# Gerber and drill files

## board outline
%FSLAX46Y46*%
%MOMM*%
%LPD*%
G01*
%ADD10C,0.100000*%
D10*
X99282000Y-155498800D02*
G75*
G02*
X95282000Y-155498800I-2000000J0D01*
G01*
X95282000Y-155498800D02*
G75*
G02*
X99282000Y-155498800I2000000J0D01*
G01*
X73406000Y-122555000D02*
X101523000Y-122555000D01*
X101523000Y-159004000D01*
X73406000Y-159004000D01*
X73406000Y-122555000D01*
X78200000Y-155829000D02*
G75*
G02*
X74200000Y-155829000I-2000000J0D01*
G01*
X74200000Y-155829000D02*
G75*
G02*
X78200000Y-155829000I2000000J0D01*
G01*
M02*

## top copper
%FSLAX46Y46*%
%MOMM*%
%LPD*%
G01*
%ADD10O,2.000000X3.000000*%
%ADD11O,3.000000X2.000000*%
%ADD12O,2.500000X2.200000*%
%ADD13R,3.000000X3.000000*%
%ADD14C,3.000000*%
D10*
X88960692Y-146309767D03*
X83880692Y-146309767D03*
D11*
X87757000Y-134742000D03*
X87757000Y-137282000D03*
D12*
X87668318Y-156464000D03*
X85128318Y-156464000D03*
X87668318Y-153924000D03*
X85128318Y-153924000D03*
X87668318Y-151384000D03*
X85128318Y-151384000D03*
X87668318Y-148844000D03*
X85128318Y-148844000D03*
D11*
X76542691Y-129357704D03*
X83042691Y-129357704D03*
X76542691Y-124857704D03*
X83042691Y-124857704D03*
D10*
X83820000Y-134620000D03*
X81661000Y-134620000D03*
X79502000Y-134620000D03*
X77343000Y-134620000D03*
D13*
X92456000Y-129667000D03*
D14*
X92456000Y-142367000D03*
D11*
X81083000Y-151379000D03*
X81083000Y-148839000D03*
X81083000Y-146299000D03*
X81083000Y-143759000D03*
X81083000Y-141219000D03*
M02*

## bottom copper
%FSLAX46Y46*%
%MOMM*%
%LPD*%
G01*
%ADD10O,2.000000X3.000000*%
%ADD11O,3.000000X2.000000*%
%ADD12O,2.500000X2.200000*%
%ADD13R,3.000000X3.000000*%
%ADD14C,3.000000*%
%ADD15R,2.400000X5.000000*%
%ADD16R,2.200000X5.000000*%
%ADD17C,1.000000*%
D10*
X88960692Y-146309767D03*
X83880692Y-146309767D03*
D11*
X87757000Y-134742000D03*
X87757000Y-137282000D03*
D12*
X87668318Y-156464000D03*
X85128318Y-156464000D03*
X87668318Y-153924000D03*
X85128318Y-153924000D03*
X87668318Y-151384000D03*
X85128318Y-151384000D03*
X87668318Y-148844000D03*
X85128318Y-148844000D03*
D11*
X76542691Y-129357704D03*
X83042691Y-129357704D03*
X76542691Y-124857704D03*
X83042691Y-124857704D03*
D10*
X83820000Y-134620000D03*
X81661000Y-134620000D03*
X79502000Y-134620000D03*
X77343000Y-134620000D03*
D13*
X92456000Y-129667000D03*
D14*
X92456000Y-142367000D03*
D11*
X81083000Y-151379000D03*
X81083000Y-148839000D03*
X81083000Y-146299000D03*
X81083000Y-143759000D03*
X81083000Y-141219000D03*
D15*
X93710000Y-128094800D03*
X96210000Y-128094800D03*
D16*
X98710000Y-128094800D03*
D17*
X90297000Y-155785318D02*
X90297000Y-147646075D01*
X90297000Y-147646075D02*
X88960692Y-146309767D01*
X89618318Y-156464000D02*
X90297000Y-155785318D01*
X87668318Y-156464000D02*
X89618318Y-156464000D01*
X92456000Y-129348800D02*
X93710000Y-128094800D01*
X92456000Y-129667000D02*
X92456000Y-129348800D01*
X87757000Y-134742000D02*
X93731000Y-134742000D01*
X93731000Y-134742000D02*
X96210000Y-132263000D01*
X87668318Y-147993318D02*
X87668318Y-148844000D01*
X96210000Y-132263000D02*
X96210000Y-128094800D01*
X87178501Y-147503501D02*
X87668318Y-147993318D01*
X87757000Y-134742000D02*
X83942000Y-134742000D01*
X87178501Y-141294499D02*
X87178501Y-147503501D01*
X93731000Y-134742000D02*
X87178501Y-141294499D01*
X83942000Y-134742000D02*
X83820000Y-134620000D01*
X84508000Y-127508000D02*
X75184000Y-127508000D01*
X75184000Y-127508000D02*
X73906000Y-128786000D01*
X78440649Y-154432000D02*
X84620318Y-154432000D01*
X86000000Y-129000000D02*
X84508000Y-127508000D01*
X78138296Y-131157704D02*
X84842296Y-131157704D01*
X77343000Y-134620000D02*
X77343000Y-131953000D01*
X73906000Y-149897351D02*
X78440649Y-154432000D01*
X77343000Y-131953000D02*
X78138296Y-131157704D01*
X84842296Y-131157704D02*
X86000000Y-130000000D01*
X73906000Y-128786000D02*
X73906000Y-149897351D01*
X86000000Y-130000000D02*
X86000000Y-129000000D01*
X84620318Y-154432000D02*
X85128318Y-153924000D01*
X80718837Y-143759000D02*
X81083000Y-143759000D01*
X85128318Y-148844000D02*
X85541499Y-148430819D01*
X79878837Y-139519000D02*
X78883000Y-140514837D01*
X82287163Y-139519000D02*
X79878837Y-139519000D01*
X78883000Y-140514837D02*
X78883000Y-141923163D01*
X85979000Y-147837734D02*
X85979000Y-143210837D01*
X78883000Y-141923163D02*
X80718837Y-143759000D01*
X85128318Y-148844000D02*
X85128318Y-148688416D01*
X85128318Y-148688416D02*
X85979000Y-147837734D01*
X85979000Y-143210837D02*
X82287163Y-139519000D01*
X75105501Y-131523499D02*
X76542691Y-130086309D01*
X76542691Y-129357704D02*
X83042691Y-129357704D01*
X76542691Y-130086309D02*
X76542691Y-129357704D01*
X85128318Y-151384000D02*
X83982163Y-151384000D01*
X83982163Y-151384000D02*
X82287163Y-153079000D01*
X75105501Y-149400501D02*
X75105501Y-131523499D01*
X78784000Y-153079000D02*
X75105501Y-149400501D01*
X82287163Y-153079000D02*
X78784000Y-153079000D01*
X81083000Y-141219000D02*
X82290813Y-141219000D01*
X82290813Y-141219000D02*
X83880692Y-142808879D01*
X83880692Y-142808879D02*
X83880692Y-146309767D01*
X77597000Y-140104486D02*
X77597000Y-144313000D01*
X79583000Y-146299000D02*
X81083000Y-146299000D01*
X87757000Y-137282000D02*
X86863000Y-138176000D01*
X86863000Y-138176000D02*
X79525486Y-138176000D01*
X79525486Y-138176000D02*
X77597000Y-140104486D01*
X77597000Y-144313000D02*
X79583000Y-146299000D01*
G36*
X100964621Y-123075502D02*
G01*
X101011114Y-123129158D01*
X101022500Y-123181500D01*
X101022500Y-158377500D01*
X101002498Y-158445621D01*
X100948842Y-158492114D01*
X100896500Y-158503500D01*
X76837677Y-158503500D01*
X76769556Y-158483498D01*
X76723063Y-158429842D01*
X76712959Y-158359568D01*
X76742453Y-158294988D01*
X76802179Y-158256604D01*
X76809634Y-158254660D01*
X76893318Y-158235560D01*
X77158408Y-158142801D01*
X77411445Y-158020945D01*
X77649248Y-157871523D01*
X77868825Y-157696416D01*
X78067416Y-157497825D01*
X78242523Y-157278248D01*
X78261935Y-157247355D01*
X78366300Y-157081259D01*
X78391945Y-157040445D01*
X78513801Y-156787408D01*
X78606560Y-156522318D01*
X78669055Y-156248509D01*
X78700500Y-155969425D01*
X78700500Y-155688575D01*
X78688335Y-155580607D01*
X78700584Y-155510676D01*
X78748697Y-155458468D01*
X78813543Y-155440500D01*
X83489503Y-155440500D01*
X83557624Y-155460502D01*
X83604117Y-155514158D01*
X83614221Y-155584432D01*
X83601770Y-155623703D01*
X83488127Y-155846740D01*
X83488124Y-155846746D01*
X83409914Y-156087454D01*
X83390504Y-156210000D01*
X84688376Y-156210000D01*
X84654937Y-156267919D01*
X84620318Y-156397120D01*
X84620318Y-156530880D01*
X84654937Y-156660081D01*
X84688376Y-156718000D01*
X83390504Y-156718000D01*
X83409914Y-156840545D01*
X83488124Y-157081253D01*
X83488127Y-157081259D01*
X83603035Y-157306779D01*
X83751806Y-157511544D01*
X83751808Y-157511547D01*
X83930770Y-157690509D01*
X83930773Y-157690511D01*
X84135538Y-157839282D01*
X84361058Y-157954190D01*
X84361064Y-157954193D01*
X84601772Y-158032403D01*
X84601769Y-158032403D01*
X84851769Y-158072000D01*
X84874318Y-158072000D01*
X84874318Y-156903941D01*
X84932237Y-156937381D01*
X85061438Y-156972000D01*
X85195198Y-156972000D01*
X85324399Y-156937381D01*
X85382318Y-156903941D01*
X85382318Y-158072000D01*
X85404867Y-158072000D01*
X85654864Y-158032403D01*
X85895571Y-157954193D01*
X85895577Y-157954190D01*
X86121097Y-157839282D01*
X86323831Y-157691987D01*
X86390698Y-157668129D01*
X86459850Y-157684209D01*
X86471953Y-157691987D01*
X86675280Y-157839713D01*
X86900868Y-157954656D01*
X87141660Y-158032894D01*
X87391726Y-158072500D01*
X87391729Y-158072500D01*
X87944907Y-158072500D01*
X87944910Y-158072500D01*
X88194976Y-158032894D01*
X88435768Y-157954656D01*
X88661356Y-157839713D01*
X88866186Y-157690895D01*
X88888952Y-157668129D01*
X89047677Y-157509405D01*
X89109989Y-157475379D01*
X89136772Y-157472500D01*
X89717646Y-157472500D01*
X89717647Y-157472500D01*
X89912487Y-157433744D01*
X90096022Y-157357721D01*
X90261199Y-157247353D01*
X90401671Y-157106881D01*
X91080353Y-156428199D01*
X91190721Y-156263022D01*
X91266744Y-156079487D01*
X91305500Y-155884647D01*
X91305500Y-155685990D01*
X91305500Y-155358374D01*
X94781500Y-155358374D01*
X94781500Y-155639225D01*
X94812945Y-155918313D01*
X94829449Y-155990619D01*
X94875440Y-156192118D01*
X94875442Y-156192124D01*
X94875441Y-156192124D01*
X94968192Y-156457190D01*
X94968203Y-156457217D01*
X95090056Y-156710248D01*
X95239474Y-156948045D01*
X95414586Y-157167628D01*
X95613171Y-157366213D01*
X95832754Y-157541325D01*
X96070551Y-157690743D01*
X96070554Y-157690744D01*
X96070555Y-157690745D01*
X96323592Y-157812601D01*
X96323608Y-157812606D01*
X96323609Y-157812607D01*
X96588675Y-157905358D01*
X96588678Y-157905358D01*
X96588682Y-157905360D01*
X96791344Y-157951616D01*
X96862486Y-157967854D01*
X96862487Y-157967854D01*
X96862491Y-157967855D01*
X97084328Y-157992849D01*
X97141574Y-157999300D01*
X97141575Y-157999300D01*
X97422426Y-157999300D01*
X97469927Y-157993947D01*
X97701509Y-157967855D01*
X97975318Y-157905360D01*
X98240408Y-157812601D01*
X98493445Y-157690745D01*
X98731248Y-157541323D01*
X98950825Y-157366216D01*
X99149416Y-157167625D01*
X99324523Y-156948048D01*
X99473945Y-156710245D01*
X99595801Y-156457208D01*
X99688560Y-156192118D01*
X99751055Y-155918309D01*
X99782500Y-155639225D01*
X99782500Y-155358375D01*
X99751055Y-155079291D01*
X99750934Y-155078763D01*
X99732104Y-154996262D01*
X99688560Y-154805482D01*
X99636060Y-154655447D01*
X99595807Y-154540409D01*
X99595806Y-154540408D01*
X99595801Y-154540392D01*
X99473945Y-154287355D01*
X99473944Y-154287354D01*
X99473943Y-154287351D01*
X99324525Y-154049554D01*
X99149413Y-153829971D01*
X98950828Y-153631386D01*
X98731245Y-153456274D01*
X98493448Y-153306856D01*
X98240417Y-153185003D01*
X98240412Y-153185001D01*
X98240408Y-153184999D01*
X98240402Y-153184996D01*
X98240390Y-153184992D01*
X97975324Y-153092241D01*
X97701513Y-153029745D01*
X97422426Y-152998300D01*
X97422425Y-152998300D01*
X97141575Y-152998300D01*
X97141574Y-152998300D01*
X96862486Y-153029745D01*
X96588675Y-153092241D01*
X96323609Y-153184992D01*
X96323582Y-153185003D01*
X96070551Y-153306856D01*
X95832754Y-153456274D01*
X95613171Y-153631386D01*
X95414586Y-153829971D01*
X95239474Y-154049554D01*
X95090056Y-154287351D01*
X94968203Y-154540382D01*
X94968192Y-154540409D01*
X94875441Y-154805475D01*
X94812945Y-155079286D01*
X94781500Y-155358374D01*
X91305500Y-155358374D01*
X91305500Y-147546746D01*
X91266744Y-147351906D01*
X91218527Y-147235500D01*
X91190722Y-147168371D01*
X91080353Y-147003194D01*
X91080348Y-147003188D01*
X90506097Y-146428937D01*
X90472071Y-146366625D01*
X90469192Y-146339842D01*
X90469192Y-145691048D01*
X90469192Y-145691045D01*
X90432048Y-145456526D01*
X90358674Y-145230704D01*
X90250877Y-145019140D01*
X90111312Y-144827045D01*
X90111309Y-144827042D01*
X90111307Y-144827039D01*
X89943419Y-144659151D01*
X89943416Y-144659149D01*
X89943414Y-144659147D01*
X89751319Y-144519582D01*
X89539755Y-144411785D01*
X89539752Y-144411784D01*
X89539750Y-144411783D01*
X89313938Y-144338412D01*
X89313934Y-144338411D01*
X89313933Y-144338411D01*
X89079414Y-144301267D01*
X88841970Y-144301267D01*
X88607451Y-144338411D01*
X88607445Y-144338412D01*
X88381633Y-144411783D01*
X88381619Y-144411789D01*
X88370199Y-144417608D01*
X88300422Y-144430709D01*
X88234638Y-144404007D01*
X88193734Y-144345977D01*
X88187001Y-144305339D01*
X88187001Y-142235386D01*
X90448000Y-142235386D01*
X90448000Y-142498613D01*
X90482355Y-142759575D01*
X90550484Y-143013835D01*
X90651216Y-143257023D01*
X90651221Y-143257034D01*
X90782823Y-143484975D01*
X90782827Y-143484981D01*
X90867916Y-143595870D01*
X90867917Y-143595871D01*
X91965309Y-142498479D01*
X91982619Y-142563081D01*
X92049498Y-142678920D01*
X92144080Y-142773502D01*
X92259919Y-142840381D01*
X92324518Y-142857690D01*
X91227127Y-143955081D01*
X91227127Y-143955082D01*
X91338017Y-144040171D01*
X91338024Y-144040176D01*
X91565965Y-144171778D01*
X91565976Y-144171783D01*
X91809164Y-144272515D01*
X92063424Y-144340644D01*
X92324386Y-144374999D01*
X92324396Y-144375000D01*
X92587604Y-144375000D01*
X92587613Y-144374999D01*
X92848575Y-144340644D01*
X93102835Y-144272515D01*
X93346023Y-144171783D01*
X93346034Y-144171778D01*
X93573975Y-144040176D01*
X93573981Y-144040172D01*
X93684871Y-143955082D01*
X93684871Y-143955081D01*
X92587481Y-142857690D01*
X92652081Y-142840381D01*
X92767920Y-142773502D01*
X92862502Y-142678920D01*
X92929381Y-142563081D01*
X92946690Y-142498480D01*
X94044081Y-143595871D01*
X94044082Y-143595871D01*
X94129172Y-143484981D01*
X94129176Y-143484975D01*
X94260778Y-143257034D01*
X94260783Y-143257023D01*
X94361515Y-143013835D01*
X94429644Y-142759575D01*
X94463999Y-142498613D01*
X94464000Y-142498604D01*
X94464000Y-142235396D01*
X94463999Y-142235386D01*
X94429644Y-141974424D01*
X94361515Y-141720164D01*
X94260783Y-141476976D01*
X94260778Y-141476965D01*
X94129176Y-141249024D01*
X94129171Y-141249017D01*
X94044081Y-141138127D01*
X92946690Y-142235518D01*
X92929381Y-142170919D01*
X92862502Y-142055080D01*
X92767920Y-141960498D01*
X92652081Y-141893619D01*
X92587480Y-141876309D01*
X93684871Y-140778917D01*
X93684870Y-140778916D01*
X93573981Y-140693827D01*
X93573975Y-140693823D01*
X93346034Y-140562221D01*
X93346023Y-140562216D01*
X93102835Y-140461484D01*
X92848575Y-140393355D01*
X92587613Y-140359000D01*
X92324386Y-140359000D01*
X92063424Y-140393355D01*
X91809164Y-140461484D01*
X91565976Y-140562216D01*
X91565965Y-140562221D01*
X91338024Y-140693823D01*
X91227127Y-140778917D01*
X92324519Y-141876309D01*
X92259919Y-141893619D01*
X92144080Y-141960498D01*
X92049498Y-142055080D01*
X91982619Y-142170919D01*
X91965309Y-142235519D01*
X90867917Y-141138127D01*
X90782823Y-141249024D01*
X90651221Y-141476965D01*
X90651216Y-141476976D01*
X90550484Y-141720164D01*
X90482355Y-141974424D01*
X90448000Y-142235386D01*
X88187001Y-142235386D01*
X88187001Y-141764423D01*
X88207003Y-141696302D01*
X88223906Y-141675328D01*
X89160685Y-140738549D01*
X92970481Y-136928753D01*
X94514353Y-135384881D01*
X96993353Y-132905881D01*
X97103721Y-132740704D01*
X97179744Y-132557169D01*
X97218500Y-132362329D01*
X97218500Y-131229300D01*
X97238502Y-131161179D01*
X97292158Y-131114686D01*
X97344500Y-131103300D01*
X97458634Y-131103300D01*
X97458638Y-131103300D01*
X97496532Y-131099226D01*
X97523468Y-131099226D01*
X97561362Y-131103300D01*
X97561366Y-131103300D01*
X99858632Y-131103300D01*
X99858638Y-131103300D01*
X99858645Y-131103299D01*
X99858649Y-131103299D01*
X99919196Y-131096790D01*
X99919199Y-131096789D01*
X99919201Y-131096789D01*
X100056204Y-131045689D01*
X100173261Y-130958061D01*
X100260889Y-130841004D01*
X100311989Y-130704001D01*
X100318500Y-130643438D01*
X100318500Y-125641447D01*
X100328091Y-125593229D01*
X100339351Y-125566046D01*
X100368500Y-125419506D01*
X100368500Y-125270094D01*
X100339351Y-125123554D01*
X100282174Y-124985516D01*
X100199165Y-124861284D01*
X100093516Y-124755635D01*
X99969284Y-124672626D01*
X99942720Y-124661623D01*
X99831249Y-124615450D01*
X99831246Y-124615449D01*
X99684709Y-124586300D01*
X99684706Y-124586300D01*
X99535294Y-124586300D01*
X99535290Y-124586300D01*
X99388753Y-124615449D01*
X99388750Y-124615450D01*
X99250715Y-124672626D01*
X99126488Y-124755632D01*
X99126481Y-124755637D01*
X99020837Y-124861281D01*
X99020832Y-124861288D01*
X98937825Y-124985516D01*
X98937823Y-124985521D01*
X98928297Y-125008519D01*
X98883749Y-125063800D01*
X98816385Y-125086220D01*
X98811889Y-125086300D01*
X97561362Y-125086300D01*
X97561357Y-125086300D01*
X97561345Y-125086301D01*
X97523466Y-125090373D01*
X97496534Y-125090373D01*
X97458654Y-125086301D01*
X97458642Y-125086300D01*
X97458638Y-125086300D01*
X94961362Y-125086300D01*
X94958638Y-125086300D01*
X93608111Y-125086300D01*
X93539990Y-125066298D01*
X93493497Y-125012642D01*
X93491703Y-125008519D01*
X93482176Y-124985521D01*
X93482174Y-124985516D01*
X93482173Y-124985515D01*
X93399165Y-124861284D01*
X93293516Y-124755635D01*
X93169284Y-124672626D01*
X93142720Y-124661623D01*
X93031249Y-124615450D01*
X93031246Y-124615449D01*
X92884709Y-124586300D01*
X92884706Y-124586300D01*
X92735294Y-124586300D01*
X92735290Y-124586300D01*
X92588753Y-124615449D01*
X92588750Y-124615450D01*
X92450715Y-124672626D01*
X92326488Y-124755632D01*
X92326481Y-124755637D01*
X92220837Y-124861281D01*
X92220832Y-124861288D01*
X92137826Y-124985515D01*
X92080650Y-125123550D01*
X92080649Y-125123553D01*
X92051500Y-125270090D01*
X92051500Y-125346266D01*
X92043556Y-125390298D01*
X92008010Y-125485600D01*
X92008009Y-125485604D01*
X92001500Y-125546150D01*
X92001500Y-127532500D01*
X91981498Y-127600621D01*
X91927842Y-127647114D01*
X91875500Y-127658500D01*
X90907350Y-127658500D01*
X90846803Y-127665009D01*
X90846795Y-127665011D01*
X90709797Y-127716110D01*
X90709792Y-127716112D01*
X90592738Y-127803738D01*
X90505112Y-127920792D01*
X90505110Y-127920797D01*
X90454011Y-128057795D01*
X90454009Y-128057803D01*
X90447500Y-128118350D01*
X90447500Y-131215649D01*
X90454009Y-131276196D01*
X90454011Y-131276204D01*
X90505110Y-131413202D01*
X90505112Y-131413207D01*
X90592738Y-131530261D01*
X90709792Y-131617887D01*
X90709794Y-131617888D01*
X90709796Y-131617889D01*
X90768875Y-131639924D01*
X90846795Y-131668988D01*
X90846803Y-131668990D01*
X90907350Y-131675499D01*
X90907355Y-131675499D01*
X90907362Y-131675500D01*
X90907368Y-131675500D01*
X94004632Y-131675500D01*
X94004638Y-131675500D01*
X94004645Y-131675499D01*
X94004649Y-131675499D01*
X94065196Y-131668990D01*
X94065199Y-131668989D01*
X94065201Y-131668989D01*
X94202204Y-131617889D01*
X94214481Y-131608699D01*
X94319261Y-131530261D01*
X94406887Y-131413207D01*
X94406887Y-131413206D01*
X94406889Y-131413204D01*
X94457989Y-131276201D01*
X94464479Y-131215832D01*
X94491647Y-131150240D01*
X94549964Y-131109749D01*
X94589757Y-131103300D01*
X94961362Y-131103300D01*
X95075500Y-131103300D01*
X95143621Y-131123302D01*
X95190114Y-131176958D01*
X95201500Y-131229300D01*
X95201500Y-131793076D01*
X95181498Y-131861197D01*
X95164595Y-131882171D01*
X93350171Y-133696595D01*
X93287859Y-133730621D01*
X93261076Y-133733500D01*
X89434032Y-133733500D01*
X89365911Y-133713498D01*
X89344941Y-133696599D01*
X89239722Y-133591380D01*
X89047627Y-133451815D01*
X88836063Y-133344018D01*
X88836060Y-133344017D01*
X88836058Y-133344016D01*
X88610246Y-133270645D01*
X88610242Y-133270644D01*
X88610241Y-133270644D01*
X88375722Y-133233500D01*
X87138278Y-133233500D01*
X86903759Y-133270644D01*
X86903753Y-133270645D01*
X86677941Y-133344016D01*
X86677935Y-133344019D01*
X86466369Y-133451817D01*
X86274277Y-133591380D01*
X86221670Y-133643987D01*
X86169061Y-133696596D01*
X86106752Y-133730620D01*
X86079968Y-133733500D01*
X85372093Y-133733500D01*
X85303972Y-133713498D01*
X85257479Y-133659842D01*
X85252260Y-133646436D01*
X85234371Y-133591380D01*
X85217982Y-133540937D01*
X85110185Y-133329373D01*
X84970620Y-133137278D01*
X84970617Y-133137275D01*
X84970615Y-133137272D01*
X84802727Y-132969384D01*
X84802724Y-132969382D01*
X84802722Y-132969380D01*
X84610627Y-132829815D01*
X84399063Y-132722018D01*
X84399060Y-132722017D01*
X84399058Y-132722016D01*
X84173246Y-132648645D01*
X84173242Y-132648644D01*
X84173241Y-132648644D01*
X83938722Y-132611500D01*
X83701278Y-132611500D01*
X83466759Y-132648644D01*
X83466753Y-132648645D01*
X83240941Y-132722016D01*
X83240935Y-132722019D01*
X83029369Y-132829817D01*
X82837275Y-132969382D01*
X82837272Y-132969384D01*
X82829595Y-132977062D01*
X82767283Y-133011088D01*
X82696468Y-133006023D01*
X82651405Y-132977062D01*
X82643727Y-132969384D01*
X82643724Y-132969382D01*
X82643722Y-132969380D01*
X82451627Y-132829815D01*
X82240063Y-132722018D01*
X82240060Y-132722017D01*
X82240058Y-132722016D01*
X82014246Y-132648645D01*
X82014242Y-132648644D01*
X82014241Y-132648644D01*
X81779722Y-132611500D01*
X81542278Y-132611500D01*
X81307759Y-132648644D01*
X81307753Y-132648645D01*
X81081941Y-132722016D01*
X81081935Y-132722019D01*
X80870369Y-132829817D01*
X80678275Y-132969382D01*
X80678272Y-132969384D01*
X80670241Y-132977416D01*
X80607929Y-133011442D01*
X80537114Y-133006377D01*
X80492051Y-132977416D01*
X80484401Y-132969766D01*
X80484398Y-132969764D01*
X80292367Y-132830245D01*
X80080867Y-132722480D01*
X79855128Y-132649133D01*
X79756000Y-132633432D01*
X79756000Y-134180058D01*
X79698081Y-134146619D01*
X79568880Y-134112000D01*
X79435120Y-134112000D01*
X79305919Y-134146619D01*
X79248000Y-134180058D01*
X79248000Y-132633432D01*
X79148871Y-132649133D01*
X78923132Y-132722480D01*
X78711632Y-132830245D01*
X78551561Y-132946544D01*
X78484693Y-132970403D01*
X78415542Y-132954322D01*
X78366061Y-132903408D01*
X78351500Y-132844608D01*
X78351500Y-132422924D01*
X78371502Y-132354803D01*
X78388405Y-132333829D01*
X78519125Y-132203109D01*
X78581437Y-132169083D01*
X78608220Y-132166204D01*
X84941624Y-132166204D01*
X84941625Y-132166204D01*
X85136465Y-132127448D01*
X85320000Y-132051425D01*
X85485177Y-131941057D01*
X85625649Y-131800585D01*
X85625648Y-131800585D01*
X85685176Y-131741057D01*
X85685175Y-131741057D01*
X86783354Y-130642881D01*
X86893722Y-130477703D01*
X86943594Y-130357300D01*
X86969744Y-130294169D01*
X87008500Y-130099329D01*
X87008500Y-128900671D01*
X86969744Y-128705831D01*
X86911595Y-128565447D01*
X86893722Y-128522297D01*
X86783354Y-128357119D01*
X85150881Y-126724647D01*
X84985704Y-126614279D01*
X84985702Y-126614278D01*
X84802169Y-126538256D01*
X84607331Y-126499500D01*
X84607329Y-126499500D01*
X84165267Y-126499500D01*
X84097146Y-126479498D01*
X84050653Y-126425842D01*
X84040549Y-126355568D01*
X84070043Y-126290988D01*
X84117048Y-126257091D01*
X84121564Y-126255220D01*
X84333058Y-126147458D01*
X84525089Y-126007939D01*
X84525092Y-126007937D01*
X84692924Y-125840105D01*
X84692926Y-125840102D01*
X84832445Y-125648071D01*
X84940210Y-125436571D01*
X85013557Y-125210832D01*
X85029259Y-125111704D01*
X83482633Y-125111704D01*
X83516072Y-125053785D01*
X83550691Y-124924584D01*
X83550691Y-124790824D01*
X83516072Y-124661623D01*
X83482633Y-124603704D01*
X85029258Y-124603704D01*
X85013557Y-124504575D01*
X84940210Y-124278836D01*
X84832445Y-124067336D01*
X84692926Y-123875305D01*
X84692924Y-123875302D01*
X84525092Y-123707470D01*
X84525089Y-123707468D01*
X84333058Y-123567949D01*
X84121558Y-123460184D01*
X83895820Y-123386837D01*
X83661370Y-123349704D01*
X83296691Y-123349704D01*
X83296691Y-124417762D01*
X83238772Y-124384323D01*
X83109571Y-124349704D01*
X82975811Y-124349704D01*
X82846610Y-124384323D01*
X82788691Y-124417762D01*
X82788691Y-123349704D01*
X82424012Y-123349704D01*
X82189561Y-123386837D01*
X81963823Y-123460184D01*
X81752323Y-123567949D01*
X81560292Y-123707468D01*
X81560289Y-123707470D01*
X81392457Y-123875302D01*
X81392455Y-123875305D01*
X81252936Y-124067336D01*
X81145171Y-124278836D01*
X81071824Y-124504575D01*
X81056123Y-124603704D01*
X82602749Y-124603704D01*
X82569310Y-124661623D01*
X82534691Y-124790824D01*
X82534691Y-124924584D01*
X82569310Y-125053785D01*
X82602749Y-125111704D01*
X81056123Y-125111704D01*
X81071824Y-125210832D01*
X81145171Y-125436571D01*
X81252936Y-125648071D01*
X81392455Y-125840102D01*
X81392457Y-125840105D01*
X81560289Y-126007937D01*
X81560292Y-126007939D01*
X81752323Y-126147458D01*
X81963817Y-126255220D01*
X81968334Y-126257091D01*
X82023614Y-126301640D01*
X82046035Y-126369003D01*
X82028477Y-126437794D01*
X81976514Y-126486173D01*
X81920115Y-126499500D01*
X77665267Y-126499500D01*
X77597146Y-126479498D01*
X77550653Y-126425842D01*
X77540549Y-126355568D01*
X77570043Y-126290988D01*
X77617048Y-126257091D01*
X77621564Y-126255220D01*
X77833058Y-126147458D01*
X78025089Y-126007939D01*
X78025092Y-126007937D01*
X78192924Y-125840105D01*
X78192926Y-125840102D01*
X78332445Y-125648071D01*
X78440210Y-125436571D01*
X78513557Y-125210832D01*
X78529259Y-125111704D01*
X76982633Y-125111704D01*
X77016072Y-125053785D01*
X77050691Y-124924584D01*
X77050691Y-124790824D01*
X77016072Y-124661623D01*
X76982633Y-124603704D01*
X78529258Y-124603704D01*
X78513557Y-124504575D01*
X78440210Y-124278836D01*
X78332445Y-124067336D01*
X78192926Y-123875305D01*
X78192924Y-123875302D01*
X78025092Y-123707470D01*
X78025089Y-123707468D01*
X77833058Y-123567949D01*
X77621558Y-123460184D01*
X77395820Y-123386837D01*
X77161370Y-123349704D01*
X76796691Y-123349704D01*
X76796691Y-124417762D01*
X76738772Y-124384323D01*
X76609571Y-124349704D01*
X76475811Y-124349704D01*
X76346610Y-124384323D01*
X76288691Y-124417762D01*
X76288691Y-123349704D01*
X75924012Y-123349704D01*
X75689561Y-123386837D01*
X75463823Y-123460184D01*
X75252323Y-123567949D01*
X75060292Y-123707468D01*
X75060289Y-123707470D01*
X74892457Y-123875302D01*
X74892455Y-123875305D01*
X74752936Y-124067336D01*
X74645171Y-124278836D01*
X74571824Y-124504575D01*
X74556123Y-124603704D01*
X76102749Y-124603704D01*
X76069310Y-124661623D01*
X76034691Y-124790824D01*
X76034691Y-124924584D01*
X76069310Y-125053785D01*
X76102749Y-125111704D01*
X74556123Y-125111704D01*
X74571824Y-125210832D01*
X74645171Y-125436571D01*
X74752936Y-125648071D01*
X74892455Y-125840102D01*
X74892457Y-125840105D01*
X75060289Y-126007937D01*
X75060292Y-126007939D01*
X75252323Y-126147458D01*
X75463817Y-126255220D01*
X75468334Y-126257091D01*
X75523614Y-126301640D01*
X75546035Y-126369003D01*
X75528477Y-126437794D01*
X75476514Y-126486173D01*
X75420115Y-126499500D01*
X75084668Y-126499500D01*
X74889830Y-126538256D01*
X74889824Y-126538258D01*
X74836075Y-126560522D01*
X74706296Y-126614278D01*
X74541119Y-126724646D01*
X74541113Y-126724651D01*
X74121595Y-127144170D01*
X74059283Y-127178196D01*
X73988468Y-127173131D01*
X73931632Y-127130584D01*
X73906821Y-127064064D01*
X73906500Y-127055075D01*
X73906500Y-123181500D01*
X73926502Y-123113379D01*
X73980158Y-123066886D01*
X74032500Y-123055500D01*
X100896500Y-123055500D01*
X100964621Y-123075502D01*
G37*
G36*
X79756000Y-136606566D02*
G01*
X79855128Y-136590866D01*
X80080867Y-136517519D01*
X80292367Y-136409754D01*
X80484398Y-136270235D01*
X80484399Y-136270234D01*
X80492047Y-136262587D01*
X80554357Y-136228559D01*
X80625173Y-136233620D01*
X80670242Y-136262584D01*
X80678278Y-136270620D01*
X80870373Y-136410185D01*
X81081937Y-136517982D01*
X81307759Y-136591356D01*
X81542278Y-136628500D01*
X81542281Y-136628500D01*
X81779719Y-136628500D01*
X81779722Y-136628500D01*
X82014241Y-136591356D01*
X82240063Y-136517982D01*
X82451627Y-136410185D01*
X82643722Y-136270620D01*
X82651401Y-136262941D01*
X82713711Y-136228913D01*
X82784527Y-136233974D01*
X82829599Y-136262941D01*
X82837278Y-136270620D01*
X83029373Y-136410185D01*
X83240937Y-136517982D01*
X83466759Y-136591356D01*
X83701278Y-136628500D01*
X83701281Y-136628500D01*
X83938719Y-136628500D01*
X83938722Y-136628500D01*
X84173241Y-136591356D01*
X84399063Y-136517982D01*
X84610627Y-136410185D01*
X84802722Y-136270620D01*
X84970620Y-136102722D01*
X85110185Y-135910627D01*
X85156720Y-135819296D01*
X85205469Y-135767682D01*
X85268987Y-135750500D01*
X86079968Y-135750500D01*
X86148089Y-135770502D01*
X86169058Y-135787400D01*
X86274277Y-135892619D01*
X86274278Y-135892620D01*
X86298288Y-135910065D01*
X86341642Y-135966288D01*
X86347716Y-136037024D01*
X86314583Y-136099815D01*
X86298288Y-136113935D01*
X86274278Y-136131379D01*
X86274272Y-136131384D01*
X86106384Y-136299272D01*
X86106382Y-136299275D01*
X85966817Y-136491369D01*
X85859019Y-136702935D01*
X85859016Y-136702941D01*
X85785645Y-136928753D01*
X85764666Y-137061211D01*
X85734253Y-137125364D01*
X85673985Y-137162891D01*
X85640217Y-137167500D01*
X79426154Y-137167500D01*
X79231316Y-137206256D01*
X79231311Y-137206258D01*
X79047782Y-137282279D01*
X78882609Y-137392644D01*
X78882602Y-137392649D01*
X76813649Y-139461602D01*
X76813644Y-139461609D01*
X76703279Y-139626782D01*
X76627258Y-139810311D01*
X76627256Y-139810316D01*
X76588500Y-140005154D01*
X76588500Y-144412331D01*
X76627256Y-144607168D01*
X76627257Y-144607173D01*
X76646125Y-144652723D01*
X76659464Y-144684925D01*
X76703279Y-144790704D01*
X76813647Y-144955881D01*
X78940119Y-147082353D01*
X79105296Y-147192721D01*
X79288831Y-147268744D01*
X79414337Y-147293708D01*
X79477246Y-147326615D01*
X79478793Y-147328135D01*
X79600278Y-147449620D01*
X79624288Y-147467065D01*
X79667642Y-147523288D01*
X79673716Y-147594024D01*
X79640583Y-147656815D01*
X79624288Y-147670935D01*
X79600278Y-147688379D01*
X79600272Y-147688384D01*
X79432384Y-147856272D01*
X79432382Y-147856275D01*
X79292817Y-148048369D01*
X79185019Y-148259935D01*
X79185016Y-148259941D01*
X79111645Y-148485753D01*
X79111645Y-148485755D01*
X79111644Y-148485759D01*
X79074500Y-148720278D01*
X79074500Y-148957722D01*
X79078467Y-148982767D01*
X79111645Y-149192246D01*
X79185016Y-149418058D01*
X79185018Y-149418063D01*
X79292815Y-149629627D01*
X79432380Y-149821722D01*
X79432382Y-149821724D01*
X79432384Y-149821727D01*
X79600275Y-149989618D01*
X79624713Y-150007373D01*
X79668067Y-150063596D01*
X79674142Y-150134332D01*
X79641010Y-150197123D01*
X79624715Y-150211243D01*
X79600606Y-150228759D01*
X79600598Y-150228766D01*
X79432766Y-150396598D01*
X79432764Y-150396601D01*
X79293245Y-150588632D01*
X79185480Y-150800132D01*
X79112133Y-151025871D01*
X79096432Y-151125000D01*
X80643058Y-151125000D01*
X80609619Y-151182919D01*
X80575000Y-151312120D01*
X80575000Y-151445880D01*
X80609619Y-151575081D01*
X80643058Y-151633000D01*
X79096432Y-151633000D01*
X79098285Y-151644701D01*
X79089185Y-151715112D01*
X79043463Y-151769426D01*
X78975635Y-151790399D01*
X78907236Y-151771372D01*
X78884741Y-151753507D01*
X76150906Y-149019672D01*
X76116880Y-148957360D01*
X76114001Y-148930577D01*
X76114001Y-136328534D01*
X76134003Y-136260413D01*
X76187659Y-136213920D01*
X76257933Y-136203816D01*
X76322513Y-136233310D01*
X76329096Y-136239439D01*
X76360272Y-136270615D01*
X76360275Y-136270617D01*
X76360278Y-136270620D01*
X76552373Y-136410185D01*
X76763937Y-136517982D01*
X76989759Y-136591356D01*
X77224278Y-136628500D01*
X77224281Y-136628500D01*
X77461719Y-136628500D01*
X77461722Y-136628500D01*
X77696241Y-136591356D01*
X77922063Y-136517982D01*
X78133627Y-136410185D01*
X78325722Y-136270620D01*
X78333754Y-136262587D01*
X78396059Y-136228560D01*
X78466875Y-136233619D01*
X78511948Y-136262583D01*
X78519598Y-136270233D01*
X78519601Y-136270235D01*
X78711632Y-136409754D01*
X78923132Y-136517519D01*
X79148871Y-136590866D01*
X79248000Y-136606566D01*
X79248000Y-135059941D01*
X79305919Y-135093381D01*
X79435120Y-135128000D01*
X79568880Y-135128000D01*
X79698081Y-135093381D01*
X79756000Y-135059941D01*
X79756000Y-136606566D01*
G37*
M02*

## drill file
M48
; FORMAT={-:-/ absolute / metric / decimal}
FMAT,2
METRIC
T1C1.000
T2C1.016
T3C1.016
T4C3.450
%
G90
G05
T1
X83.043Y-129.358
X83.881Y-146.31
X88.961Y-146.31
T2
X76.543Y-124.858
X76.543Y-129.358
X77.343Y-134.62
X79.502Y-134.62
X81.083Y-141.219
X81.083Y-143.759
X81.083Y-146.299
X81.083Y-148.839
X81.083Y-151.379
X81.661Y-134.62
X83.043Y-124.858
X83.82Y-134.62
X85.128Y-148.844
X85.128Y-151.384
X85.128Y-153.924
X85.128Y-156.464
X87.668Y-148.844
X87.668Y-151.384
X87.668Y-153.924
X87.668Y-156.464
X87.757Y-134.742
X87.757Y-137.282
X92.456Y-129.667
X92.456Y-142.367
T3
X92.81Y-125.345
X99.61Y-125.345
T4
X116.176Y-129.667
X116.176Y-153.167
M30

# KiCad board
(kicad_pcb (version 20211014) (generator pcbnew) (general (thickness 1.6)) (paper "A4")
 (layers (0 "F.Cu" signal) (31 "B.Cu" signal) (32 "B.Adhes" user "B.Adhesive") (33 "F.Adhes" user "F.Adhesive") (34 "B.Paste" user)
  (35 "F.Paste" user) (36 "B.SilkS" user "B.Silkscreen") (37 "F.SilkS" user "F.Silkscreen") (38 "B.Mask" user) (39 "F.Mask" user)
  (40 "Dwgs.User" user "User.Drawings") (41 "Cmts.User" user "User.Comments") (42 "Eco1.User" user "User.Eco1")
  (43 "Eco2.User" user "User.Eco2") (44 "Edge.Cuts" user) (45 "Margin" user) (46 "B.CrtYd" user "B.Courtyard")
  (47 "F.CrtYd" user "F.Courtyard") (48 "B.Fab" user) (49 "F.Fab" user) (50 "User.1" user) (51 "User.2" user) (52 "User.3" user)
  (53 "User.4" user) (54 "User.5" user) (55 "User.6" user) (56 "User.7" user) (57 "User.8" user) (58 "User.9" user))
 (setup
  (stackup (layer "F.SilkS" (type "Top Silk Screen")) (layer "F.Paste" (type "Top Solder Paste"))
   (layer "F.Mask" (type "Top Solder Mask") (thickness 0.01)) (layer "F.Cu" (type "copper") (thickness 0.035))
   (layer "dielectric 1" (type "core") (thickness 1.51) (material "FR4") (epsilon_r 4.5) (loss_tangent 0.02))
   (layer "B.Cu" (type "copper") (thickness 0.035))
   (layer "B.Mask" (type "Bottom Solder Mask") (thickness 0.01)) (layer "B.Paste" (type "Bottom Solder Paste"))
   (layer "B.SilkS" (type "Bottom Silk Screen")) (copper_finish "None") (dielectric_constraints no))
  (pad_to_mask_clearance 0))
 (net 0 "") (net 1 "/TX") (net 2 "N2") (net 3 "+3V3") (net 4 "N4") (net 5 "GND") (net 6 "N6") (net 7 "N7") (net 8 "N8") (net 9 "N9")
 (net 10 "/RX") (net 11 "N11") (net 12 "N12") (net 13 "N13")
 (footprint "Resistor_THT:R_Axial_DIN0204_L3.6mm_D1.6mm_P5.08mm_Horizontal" (layer "F.Cu") (at 88.960692 146.309767 180)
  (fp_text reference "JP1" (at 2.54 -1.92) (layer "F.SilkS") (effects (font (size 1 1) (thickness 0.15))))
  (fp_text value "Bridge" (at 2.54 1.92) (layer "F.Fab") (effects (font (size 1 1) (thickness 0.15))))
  (pad "1" thru_hole oval (at 0 0 270) (size 3 2) (drill 1) (layers *.Cu *.Mask) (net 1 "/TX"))
  (pad "2" thru_hole oval (at 5.08 0 270) (size 3 2) (drill 1) (layers *.Cu *.Mask) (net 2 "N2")))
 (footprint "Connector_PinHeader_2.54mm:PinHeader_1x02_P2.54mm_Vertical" (layer "F.Cu") (at 87.757 134.742)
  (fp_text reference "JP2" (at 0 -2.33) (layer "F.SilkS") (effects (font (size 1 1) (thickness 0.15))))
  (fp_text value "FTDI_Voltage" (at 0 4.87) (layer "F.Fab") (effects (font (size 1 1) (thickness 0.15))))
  (pad "1" thru_hole oval (at 0 0) (size 3 2) (drill 1.016) (layers *.Cu *.Mask) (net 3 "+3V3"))
  (pad "2" thru_hole oval (at 0 2.54) (size 3 2) (drill 1.016) (layers *.Cu *.Mask) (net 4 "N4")))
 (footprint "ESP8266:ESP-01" (layer "F.Cu") (at 87.668318 156.464 180)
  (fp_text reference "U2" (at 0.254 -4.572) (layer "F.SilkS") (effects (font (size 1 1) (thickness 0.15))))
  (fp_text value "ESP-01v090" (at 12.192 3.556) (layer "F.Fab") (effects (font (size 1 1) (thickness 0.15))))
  (pad "1" thru_hole oval (at 0 0 180) (size 2.5 2.2) (drill 1.016) (layers *.Cu *.Mask "F.SilkS") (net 1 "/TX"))
  (pad "2" thru_hole oval (at 2.54 0 180) (size 2.5 2.2) (drill 1.016) (layers *.Cu *.Mask "F.SilkS") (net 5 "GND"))
  (pad "3" thru_hole oval (at 0 2.54 180) (size 2.5 2.2) (drill 1.016) (layers *.Cu *.Mask "F.SilkS") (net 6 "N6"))
  (pad "4" thru_hole oval (at 2.54 2.54 180) (size 2.5 2.2) (drill 1.016) (layers *.Cu *.Mask "F.SilkS") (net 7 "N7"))
  (pad "5" thru_hole oval (at 0 5.08 180) (size 2.5 2.2) (drill 1.016) (layers *.Cu *.Mask "F.SilkS") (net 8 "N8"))
  (pad "6" thru_hole oval (at 2.54 5.08 180) (size 2.5 2.2) (drill 1.016) (layers *.Cu *.Mask "F.SilkS") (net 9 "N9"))
  (pad "7" thru_hole oval (at 0 7.62 180) (size 2.5 2.2) (drill 1.016) (layers *.Cu *.Mask "F.SilkS") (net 3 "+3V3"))
  (pad "8" thru_hole oval (at 2.54 7.62 180) (size 2.5 2.2) (drill 1.016) (layers *.Cu *.Mask "F.SilkS") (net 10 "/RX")))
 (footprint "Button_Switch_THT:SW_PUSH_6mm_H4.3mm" (layer "F.Cu") (at 83.042691 129.357704 180)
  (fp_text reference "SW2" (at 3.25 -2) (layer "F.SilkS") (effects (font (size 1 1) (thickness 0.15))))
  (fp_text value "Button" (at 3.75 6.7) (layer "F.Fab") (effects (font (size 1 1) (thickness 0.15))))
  (pad "1" thru_hole oval (at 6.5 0 270) (size 2 3) (drill 1.016) (layers *.Cu *.Mask) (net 9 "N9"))
  (pad "1" thru_hole oval (at 0 0 270) (size 2 3) (drill 1) (layers *.Cu *.Mask) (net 9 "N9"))
  (pad "2" thru_hole oval (at 6.5 4.5 270) (size 2 3) (drill 1.016) (layers *.Cu *.Mask) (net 5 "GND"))
  (pad "2" thru_hole oval (at 0 4.5 270) (size 2 3) (drill 1.016) (layers *.Cu *.Mask) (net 5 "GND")))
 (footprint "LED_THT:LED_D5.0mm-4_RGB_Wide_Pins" (layer "F.Cu") (at 83.82 134.62 180)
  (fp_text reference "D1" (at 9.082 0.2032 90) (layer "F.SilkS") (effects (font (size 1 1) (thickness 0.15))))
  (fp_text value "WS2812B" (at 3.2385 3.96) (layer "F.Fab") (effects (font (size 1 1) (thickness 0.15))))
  (pad "1" thru_hole oval (at 0 0 270) (size 3 2) (drill 1.016) (layers *.Cu *.Mask) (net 3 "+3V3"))
  (pad "2" thru_hole oval (at 2.159 0 270) (size 3 2) (drill 1.016) (layers *.Cu *.Mask) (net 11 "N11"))
  (pad "3" thru_hole oval (at 4.318 0 270) (size 3 2) (drill 1.016) (layers *.Cu *.Mask) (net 5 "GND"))
  (pad "4" thru_hole oval (at 6.477 0 270) (size 3 2) (drill 1.016) (layers *.Cu *.Mask) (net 7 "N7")))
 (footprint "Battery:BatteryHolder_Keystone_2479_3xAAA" (layer "F.Cu") (at 92.456 129.667)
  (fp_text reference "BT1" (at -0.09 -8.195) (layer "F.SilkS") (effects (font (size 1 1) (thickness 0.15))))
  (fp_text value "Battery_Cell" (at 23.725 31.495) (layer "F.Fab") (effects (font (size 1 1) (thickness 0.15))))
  (pad "" np_thru_hole circle (at 23.72 0) (size 3.45 3.45) (drill 3.45) (layers *.Cu *.Mask))
  (pad "" np_thru_hole circle (at 23.72 23.5) (size 3.45 3.45) (drill 3.45) (layers *.Cu *.Mask))
  (pad "1" thru_hole rect (at 0 0) (size 3 3) (drill 1.016) (layers *.Cu *.Mask) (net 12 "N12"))
  (pad "2" thru_hole circle (at 0 12.7) (size 3 3) (drill 1.016) (layers *.Cu *.Mask) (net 5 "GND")))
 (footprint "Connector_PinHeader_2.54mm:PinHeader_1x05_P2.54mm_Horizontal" (layer "F.Cu") (at 81.083 151.379 180)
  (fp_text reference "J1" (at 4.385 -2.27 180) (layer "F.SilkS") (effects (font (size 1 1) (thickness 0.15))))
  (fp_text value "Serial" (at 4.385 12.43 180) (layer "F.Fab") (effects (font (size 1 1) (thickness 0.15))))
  (pad "1" thru_hole oval (at 0 0 180) (size 3 2) (drill 1.016) (layers *.Cu *.Mask) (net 5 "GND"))
  (pad "2" thru_hole oval (at 0 2.54 180) (size 3 2) (drill 1.016) (layers *.Cu *.Mask) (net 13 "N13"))
  (pad "3" thru_hole oval (at 0 5.08 180) (size 3 2) (drill 1.016) (layers *.Cu *.Mask) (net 4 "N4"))
  (pad "4" thru_hole oval (at 0 7.62 180) (size 3 2) (drill 1.016) (layers *.Cu *.Mask) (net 10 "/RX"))
  (pad "5" thru_hole oval (at 0 10.16 180) (size 3 2) (drill 1.016) (layers *.Cu *.Mask) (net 2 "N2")))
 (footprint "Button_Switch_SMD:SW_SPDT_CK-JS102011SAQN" (layer "B.Cu") (at 96.21 125.3448)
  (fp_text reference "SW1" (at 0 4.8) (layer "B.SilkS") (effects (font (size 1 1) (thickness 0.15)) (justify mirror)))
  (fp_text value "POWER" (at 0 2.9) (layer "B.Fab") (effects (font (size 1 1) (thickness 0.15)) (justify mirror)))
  (pad "" np_thru_hole circle (at -3.4 0) (size 0.9 0.9) (drill 1.016) (layers F&B.Cu *.Mask))
  (pad "" np_thru_hole circle (at 3.4 0) (size 0.9 0.9) (drill 1.016) (layers F&B.Cu *.Mask))
  (pad "1" smd rect (at -2.5 2.75) (size 2.4 5) (layers "B.Cu" "B.Paste" "B.Mask") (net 12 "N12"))
  (pad "2" smd rect (at 0 2.75) (size 2.4 5) (layers "B.Cu" "B.Paste" "B.Mask") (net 3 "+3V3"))
  (pad "3" smd rect (at 2.5 2.75) (size 2.2 5) (layers "B.Cu" "B.Paste" "B.Mask")))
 (gr_circle (center 97.282 155.4988) (end 99.282 155.4988) (layer "Edge.Cuts") (width 0.1) (fill none))
 (gr_rect (start 73.406 122.555) (end 101.523 159.004) (layer "Edge.Cuts") (width 0.1) (fill none))
 (gr_circle (center 76.2 155.829) (end 78.2 155.829) (layer "Edge.Cuts") (width 0.1) (fill none))
 (segment (start 90.297 155.785318) (end 90.297 147.646075) (width 1) (layer "B.Cu") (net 1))
 (segment (start 90.297 147.646075) (end 88.960692 146.309767) (width 1) (layer "B.Cu") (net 1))
 (segment (start 89.618318 156.464) (end 90.297 155.785318) (width 1) (layer "B.Cu") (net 1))
 (segment (start 87.668318 156.464) (end 89.618318 156.464) (width 1) (layer "B.Cu") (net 1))
 (segment (start 92.456 129.3488) (end 93.71 128.0948) (width 1) (layer "B.Cu") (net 12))
 (segment (start 92.456 129.667) (end 92.456 129.3488) (width 1) (layer "B.Cu") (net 12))
 (segment (start 87.757 134.742) (end 93.731 134.742) (width 1) (layer "B.Cu") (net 3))
 (segment (start 93.731 134.742) (end 96.21 132.263) (width 1) (layer "B.Cu") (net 3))
 (segment (start 87.668318 147.993318) (end 87.668318 148.844) (width 1) (layer "B.Cu") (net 3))
 (segment (start 96.21 132.263) (end 96.21 128.0948) (width 1) (layer "B.Cu") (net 3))
 (segment (start 87.178501 147.503501) (end 87.668318 147.993318) (width 1) (layer "B.Cu") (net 3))
 (segment (start 87.757 134.742) (end 83.942 134.742) (width 1) (layer "B.Cu") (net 3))
 (segment (start 87.178501 141.294499) (end 87.178501 147.503501) (width 1) (layer "B.Cu") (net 3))
 (segment (start 93.731 134.742) (end 87.178501 141.294499) (width 1) (layer "B.Cu") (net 3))
 (segment (start 83.942 134.742) (end 83.82 134.62) (width 1) (layer "B.Cu") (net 3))
 (segment (start 84.508 127.508) (end 75.184 127.508) (width 1) (layer "B.Cu") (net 7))
 (segment (start 75.184 127.508) (end 73.906 128.786) (width 1) (layer "B.Cu") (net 7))
 (segment (start 78.440649 154.432) (end 84.620318 154.432) (width 1) (layer "B.Cu") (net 7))
 (segment (start 86 129) (end 84.508 127.508) (width 1) (layer "B.Cu") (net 7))
 (segment (start 78.138296 131.157704) (end 84.842296 131.157704) (width 1) (layer "B.Cu") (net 7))
 (segment (start 77.343 134.62) (end 77.343 131.953) (width 1) (layer "B.Cu") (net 7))
 (segment (start 73.906 149.897351) (end 78.440649 154.432) (width 1) (layer "B.Cu") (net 7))
 (segment (start 77.343 131.953) (end 78.138296 131.157704) (width 1) (layer "B.Cu") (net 7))
 (segment (start 84.842296 131.157704) (end 86 130) (width 1) (layer "B.Cu") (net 7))
 (segment (start 73.906 128.786) (end 73.906 149.897351) (width 1) (layer "B.Cu") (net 7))
 (segment (start 86 130) (end 86 129) (width 1) (layer "B.Cu") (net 7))
 (segment (start 84.620318 154.432) (end 85.128318 153.924) (width 1) (layer "B.Cu") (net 7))
 (segment (start 80.718837 143.759) (end 81.083 143.759) (width 1) (layer "B.Cu") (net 10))
 (segment (start 85.128318 148.844) (end 85.541499 148.430819) (width 1) (layer "B.Cu") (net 10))
 (segment (start 79.878837 139.519) (end 78.883 140.514837) (width 1) (layer "B.Cu") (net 10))
 (segment (start 82.287163 139.519) (end 79.878837 139.519) (width 1) (layer "B.Cu") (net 10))
 (segment (start 78.883 140.514837) (end 78.883 141.923163) (width 1) (layer "B.Cu") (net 10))
 (segment (start 85.979 147.837734) (end 85.979 143.210837) (width 1) (layer "B.Cu") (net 10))
 (segment (start 78.883 141.923163) (end 80.718837 143.759) (width 1) (layer "B.Cu") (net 10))
 (segment (start 85.128318 148.844) (end 85.128318 148.688416) (width 1) (layer "B.Cu") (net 10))
 (segment (start 85.128318 148.688416) (end 85.979 147.837734) (width 1) (layer "B.Cu") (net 10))
 (segment (start 85.979 143.210837) (end 82.287163 139.519) (width 1) (layer "B.Cu") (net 10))
 (segment (start 75.105501 131.523499) (end 76.542691 130.086309) (width 1) (layer "B.Cu") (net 9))
 (segment (start 76.542691 129.357704) (end 83.042691 129.357704) (width 1) (layer "B.Cu") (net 9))
 (segment (start 76.542691 130.086309) (end 76.542691 129.357704) (width 1) (layer "B.Cu") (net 9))
 (segment (start 85.128318 151.384) (end 83.982163 151.384) (width 1) (layer "B.Cu") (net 9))
 (segment (start 83.982163 151.384) (end 82.287163 153.079) (width 1) (layer "B.Cu") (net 9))
 (segment (start 75.105501 149.400501) (end 75.105501 131.523499) (width 1) (layer "B.Cu") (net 9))
 (segment (start 78.784 153.079) (end 75.105501 149.400501) (width 1) (layer "B.Cu") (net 9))
 (segment (start 82.287163 153.079) (end 78.784 153.079) (width 1) (layer "B.Cu") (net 9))
 (segment (start 81.083 141.219) (end 82.290813 141.219) (width 1) (layer "B.Cu") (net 2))
 (segment (start 82.290813 141.219) (end 83.880692 142.808879) (width 1) (layer "B.Cu") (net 2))
 (segment (start 83.880692 142.808879) (end 83.880692 146.309767) (width 1) (layer "B.Cu") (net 2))
 (segment (start 77.597 140.104486) (end 77.597 144.313) (width 1) (layer "B.Cu") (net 4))
 (segment (start 79.583 146.299) (end 81.083 146.299) (width 1) (layer "B.Cu") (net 4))
 (segment (start 87.757 137.282) (end 86.863 138.176) (width 1) (layer "B.Cu") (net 4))
 (segment (start 86.863 138.176) (end 79.525486 138.176) (width 1) (layer "B.Cu") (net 4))
 (segment (start 79.525486 138.176) (end 77.597 140.104486) (width 1) (layer "B.Cu") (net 4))
 (segment (start 77.597 144.313) (end 79.583 146.299) (width 1) (layer "B.Cu") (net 4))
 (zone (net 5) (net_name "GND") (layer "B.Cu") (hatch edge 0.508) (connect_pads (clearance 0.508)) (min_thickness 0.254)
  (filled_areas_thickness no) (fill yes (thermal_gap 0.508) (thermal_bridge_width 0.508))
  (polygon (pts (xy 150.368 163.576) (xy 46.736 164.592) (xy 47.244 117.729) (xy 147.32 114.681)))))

